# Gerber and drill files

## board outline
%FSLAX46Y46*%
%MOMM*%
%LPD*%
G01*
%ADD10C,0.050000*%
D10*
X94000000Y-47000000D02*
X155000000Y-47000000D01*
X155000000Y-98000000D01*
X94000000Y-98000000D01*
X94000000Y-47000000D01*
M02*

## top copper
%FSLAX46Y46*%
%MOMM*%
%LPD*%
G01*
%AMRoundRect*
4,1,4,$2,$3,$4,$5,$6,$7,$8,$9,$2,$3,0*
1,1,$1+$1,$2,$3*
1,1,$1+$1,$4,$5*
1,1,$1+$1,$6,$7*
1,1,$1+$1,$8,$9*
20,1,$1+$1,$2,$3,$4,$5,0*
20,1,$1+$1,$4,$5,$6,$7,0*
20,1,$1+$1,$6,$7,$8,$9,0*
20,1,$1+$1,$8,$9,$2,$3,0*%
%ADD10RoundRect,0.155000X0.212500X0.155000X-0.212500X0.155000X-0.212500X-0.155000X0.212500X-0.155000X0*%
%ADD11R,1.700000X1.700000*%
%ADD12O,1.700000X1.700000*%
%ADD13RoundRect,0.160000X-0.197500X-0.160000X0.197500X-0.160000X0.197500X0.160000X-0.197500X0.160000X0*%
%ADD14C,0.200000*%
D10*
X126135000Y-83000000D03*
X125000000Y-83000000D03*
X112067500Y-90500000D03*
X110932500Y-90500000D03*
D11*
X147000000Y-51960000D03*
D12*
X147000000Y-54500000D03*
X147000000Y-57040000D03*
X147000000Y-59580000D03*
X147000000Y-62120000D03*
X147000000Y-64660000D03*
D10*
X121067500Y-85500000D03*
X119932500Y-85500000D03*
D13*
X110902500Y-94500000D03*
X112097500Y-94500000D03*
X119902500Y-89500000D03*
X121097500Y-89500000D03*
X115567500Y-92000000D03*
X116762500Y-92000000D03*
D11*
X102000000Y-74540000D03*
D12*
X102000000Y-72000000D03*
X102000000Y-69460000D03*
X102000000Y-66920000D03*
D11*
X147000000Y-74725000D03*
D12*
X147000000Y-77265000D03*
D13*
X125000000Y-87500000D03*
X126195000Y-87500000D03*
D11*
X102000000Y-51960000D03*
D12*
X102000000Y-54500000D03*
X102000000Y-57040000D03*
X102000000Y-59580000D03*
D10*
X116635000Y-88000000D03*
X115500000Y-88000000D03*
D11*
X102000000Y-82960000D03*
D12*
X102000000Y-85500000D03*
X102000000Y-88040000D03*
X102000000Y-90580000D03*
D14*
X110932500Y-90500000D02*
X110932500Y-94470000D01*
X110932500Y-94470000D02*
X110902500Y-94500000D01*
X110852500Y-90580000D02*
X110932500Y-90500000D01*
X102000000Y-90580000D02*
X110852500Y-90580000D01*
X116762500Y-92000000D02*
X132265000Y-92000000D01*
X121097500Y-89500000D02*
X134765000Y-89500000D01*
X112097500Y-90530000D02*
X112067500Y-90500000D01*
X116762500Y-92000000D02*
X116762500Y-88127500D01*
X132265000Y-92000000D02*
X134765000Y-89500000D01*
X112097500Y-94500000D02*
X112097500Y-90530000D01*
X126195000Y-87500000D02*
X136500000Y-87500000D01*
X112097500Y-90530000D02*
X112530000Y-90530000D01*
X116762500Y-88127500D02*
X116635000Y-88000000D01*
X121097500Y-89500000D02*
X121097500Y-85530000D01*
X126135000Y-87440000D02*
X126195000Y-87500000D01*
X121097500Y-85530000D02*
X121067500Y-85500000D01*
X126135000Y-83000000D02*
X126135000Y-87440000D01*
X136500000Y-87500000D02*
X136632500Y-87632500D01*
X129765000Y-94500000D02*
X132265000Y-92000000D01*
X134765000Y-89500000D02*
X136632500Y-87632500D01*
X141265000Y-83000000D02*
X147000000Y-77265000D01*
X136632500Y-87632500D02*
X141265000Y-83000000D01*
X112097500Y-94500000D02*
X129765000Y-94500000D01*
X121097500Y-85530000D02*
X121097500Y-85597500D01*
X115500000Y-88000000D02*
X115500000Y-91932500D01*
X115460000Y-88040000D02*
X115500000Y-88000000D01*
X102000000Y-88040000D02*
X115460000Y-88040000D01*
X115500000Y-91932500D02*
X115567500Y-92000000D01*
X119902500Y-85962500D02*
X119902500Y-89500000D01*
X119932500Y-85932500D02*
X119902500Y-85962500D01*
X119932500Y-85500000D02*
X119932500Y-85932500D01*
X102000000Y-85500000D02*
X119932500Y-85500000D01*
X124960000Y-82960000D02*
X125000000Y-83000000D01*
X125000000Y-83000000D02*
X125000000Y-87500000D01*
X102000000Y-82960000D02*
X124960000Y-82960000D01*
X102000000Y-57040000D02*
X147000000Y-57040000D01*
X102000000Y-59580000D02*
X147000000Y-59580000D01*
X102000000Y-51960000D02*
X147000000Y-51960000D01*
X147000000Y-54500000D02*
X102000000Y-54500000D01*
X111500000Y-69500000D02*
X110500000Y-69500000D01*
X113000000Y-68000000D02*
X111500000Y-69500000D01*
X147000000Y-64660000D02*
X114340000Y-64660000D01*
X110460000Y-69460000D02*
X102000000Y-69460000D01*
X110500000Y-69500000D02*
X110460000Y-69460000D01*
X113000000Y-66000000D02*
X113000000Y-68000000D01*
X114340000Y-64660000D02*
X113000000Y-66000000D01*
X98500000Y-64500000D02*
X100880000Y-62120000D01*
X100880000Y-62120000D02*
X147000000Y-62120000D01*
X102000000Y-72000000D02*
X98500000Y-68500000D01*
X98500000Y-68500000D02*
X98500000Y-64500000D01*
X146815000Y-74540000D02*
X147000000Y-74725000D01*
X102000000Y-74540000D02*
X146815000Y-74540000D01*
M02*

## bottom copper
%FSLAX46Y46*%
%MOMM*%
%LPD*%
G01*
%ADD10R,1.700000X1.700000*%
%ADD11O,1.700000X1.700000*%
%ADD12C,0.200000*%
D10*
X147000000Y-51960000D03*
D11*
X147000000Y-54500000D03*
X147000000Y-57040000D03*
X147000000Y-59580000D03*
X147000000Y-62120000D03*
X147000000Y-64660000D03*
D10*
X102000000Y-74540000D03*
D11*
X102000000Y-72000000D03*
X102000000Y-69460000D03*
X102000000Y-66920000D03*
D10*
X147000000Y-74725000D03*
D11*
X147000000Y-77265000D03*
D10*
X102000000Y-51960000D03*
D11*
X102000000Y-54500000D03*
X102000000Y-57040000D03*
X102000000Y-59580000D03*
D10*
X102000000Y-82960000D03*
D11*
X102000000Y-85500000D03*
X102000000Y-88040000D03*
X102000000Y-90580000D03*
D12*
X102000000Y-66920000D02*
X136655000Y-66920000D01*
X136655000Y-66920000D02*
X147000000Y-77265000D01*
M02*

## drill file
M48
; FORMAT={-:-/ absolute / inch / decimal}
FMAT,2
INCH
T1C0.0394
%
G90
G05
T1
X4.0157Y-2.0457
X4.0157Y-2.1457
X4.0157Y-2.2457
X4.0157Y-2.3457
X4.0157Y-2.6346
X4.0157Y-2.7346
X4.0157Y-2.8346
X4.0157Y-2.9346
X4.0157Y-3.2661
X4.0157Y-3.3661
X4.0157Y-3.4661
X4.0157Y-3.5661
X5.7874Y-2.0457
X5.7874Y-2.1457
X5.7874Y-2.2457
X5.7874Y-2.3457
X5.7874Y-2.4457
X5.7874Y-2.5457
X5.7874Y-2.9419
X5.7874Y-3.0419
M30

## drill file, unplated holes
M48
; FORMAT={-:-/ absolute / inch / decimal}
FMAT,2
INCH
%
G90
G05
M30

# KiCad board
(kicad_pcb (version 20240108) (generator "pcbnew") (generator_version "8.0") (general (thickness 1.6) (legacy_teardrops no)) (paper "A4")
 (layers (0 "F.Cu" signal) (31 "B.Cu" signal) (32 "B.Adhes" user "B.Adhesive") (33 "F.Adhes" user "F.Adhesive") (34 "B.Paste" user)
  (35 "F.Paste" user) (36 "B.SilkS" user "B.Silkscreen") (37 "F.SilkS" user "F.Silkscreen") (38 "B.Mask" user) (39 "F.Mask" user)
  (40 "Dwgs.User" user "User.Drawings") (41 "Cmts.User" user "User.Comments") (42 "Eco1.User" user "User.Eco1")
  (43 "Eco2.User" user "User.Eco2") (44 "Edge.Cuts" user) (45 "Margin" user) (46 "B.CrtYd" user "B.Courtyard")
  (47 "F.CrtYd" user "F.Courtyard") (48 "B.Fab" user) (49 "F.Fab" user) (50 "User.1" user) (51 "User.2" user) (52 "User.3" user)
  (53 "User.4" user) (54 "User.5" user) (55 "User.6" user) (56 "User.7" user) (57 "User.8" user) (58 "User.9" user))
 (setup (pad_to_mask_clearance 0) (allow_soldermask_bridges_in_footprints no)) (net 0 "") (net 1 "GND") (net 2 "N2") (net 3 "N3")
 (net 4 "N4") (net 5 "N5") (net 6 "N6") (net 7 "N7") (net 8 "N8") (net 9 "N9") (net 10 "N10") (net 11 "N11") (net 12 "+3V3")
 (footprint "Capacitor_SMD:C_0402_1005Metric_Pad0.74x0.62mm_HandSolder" (layer "F.Cu") (at 125.5675 83 180)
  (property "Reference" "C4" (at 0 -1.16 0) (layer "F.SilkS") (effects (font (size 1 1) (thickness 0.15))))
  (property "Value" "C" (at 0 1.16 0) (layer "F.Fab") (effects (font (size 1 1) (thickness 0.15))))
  (pad "1" smd roundrect (at -0.5675 0 180) (size 0.735 0.62) (layers "F.Cu" "F.Paste" "F.Mask") (roundrect_rratio 0.25) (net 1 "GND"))
  (pad "2" smd roundrect (at 0.5675 0 180) (size 0.735 0.62) (layers "F.Cu" "F.Paste" "F.Mask") (roundrect_rratio 0.25) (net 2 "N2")))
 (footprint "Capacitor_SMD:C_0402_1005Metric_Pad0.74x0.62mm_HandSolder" (layer "F.Cu") (at 111.5 90.5 180)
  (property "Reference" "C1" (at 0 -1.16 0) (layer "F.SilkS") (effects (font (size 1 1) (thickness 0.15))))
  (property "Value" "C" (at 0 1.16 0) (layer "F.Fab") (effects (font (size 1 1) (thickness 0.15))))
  (pad "1" smd roundrect (at -0.5675 0 180) (size 0.735 0.62) (layers "F.Cu" "F.Paste" "F.Mask") (roundrect_rratio 0.25) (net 1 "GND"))
  (pad "2" smd roundrect (at 0.5675 0 180) (size 0.735 0.62) (layers "F.Cu" "F.Paste" "F.Mask") (roundrect_rratio 0.25) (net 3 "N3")))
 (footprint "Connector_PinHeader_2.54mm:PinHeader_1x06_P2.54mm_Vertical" (layer "F.Cu") (at 147 51.96)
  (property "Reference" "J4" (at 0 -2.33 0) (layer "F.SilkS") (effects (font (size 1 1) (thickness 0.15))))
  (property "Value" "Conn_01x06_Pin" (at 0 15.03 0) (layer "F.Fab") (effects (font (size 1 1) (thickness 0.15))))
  (pad "1" thru_hole rect (at 0 0) (size 1.7 1.7) (drill 1) (layers "*.Cu" "*.Mask") (remove_unused_layers no) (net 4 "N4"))
  (pad "2" thru_hole oval (at 0 2.54) (size 1.7 1.7) (drill 1) (layers "*.Cu" "*.Mask") (remove_unused_layers no) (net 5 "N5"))
  (pad "3" thru_hole oval (at 0 5.08) (size 1.7 1.7) (drill 1) (layers "*.Cu" "*.Mask") (remove_unused_layers no) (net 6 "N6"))
  (pad "4" thru_hole oval (at 0 7.62) (size 1.7 1.7) (drill 1) (layers "*.Cu" "*.Mask") (remove_unused_layers no) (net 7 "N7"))
  (pad "5" thru_hole oval (at 0 10.16) (size 1.7 1.7) (drill 1) (layers "*.Cu" "*.Mask") (remove_unused_layers no) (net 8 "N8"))
  (pad "6" thru_hole oval (at 0 12.7) (size 1.7 1.7) (drill 1) (layers "*.Cu" "*.Mask") (remove_unused_layers no) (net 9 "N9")))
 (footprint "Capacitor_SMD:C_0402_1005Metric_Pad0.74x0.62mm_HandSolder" (layer "F.Cu") (at 120.5 85.5 180)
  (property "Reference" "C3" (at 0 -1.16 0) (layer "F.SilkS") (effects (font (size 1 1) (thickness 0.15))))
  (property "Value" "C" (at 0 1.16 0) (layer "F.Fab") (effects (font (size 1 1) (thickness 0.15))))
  (pad "1" smd roundrect (at -0.5675 0 180) (size 0.735 0.62) (layers "F.Cu" "F.Paste" "F.Mask") (roundrect_rratio 0.25) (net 1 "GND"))
  (pad "2" smd roundrect (at 0.5675 0 180) (size 0.735 0.62) (layers "F.Cu" "F.Paste" "F.Mask") (roundrect_rratio 0.25) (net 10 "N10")))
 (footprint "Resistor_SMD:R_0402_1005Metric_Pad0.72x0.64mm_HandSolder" (layer "F.Cu") (at 111.5 94.5)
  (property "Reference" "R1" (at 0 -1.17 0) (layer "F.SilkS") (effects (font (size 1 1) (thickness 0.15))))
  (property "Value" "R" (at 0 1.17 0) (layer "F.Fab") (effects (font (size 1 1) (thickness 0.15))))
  (pad "1" smd roundrect (at -0.5975 0) (size 0.715 0.64) (layers "F.Cu" "F.Paste" "F.Mask") (roundrect_rratio 0.25) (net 3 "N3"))
  (pad "2" smd roundrect (at 0.5975 0) (size 0.715 0.64) (layers "F.Cu" "F.Paste" "F.Mask") (roundrect_rratio 0.25) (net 1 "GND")))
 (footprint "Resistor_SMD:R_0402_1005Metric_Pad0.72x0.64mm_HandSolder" (layer "F.Cu") (at 120.5 89.5)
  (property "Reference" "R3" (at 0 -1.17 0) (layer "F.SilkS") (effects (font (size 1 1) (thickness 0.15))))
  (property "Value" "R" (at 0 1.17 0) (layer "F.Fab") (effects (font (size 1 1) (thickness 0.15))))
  (pad "1" smd roundrect (at -0.5975 0) (size 0.715 0.64) (layers "F.Cu" "F.Paste" "F.Mask") (roundrect_rratio 0.25) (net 10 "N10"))
  (pad "2" smd roundrect (at 0.5975 0) (size 0.715 0.64) (layers "F.Cu" "F.Paste" "F.Mask") (roundrect_rratio 0.25) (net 1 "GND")))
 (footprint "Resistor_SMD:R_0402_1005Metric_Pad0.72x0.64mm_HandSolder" (layer "F.Cu") (at 116.165 92)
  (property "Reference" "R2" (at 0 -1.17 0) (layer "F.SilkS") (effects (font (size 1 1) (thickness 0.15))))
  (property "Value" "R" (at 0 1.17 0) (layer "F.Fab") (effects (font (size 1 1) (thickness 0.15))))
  (pad "1" smd roundrect (at -0.5975 0) (size 0.715 0.64) (layers "F.Cu" "F.Paste" "F.Mask") (roundrect_rratio 0.25) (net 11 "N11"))
  (pad "2" smd roundrect (at 0.5975 0) (size 0.715 0.64) (layers "F.Cu" "F.Paste" "F.Mask") (roundrect_rratio 0.25) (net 1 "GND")))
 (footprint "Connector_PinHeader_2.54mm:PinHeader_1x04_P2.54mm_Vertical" (layer "F.Cu") (at 102 74.54 180)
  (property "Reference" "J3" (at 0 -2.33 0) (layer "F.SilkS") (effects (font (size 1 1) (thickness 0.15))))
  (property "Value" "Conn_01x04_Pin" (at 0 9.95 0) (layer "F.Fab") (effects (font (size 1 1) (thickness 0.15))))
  (pad "1" thru_hole rect (at 0 0 180) (size 1.7 1.7) (drill 1) (layers "*.Cu" "*.Mask") (remove_unused_layers no) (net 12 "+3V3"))
  (pad "2" thru_hole oval (at 0 2.54 180) (size 1.7 1.7) (drill 1) (layers "*.Cu" "*.Mask") (remove_unused_layers no) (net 8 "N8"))
  (pad "3" thru_hole oval (at 0 5.08 180) (size 1.7 1.7) (drill 1) (layers "*.Cu" "*.Mask") (remove_unused_layers no) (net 9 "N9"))
  (pad "4" thru_hole oval (at 0 7.62 180) (size 1.7 1.7) (drill 1) (layers "*.Cu" "*.Mask") (remove_unused_layers no) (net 1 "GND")))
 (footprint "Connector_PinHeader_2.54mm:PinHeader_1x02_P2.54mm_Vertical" (layer "F.Cu") (at 147 74.725)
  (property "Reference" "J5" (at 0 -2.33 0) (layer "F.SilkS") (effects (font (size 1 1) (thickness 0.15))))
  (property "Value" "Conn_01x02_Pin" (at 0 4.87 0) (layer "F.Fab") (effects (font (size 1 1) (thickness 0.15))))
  (pad "1" thru_hole rect (at 0 0) (size 1.7 1.7) (drill 1) (layers "*.Cu" "*.Mask") (remove_unused_layers no) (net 12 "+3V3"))
  (pad "2" thru_hole oval (at 0 2.54) (size 1.7 1.7) (drill 1) (layers "*.Cu" "*.Mask") (remove_unused_layers no) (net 1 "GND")))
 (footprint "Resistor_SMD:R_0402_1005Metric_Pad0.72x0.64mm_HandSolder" (layer "F.Cu") (at 125.5975 87.5)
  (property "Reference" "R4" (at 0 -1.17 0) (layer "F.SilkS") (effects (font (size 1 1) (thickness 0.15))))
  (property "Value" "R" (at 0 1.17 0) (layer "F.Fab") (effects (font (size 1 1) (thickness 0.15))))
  (pad "1" smd roundrect (at -0.5975 0) (size 0.715 0.64) (layers "F.Cu" "F.Paste" "F.Mask") (roundrect_rratio 0.25) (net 2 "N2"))
  (pad "2" smd roundrect (at 0.5975 0) (size 0.715 0.64) (layers "F.Cu" "F.Paste" "F.Mask") (roundrect_rratio 0.25) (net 1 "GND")))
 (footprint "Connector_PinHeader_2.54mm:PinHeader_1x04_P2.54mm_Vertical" (layer "F.Cu") (at 102 51.96)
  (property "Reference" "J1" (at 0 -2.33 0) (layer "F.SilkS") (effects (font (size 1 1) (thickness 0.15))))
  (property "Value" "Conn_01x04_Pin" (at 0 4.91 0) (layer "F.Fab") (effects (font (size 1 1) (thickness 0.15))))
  (pad "1" thru_hole rect (at 0 0) (size 1.7 1.7) (drill 1) (layers "*.Cu" "*.Mask") (remove_unused_layers no) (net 4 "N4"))
  (pad "2" thru_hole oval (at 0 2.54) (size 1.7 1.7) (drill 1) (layers "*.Cu" "*.Mask") (remove_unused_layers no) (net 5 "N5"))
  (pad "3" thru_hole oval (at 0 5.08) (size 1.7 1.7) (drill 1) (layers "*.Cu" "*.Mask") (remove_unused_layers no) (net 6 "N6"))
  (pad "4" thru_hole oval (at 0 7.62) (size 1.7 1.7) (drill 1) (layers "*.Cu" "*.Mask") (remove_unused_layers no) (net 7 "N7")))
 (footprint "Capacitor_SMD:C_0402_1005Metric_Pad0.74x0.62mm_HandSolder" (layer "F.Cu") (at 116.0675 88 180)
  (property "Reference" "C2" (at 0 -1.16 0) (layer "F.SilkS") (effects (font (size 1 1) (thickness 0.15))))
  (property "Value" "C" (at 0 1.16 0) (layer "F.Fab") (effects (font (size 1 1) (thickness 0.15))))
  (pad "1" smd roundrect (at -0.5675 0 180) (size 0.735 0.62) (layers "F.Cu" "F.Paste" "F.Mask") (roundrect_rratio 0.25) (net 1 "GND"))
  (pad "2" smd roundrect (at 0.5675 0 180) (size 0.735 0.62) (layers "F.Cu" "F.Paste" "F.Mask") (roundrect_rratio 0.25) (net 11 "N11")))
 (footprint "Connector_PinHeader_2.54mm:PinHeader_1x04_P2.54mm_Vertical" (layer "F.Cu") (at 102 82.96)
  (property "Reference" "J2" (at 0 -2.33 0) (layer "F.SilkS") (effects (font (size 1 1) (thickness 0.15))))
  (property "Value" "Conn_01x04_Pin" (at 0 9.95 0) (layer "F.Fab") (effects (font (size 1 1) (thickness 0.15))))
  (pad "1" thru_hole rect (at 0 0) (size 1.7 1.7) (drill 1) (layers "*.Cu" "*.Mask") (remove_unused_layers no) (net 2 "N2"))
  (pad "2" thru_hole oval (at 0 2.54) (size 1.7 1.7) (drill 1) (layers "*.Cu" "*.Mask") (remove_unused_layers no) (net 10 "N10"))
  (pad "3" thru_hole oval (at 0 5.08) (size 1.7 1.7) (drill 1) (layers "*.Cu" "*.Mask") (remove_unused_layers no) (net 11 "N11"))
  (pad "4" thru_hole oval (at 0 7.62) (size 1.7 1.7) (drill 1) (layers "*.Cu" "*.Mask") (remove_unused_layers no) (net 3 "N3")))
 (gr_rect (start 94 47) (end 155 98) (stroke (width 0.05) (type default)) (fill none) (layer "Edge.Cuts"))
 (segment (start 110.9325 90.5) (end 110.9325 94.47) (width 0.2) (layer "F.Cu") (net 3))
 (segment (start 110.9325 94.47) (end 110.9025 94.5) (width 0.2) (layer "F.Cu") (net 3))
 (segment (start 110.8525 90.58) (end 110.9325 90.5) (width 0.2) (layer "F.Cu") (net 3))
 (segment (start 102 90.58) (end 110.8525 90.58) (width 0.2) (layer "F.Cu") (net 3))
 (segment (start 116.7625 92) (end 132.265 92) (width 0.2) (layer "F.Cu") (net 1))
 (segment (start 121.0975 89.5) (end 134.765 89.5) (width 0.2) (layer "F.Cu") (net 1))
 (segment (start 112.0975 90.53) (end 112.0675 90.5) (width 0.2) (layer "F.Cu") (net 1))
 (segment (start 116.7625 92) (end 116.7625 88.1275) (width 0.2) (layer "F.Cu") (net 1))
 (segment (start 132.265 92) (end 134.765 89.5) (width 0.2) (layer "F.Cu") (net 1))
 (segment (start 112.0975 94.5) (end 112.0975 90.53) (width 0.2) (layer "F.Cu") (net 1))
 (segment (start 126.195 87.5) (end 136.5 87.5) (width 0.2) (layer "F.Cu") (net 1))
 (segment (start 112.0975 90.53) (end 112.53 90.53) (width 0.2) (layer "F.Cu") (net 1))
 (segment (start 116.7625 88.1275) (end 116.635 88) (width 0.2) (layer "F.Cu") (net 1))
 (segment (start 121.0975 89.5) (end 121.0975 85.53) (width 0.2) (layer "F.Cu") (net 1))
 (segment (start 126.135 87.44) (end 126.195 87.5) (width 0.2) (layer "F.Cu") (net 1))
 (segment (start 121.0975 85.53) (end 121.0675 85.5) (width 0.2) (layer "F.Cu") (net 1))
 (segment (start 126.135 83) (end 126.135 87.44) (width 0.2) (layer "F.Cu") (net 1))
 (segment (start 136.5 87.5) (end 136.6325 87.6325) (width 0.2) (layer "F.Cu") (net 1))
 (segment (start 129.765 94.5) (end 132.265 92) (width 0.2) (layer "F.Cu") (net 1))
 (segment (start 134.765 89.5) (end 136.6325 87.6325) (width 0.2) (layer "F.Cu") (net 1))
 (segment (start 141.265 83) (end 147 77.265) (width 0.2) (layer "F.Cu") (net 1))
 (segment (start 136.6325 87.6325) (end 141.265 83) (width 0.2) (layer "F.Cu") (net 1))
 (segment (start 112.0975 94.5) (end 129.765 94.5) (width 0.2) (layer "F.Cu") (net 1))
 (segment (start 121.0975 85.53) (end 121.0975 85.5975) (width 0.2) (layer "F.Cu") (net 1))
 (segment (start 102 66.92) (end 136.655 66.92) (width 0.2) (layer "B.Cu") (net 1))
 (segment (start 136.655 66.92) (end 147 77.265) (width 0.2) (layer "B.Cu") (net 1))
 (segment (start 115.5 88) (end 115.5 91.9325) (width 0.2) (layer "F.Cu") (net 11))
 (segment (start 115.46 88.04) (end 115.5 88) (width 0.2) (layer "F.Cu") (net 11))
 (segment (start 102 88.04) (end 115.46 88.04) (width 0.2) (layer "F.Cu") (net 11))
 (segment (start 115.5 91.9325) (end 115.5675 92) (width 0.2) (layer "F.Cu") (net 11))
 (segment (start 119.9025 85.9625) (end 119.9025 89.5) (width 0.2) (layer "F.Cu") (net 10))
 (segment (start 119.9325 85.9325) (end 119.9025 85.9625) (width 0.2) (layer "F.Cu") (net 10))
 (segment (start 119.9325 85.5) (end 119.9325 85.9325) (width 0.2) (layer "F.Cu") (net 10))
 (segment (start 102 85.5) (end 119.9325 85.5) (width 0.2) (layer "F.Cu") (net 10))
 (segment (start 124.96 82.96) (end 125 83) (width 0.2) (layer "F.Cu") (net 2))
 (segment (start 125 83) (end 125 87.5) (width 0.2) (layer "F.Cu") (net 2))
 (segment (start 102 82.96) (end 124.96 82.96) (width 0.2) (layer "F.Cu") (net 2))
 (segment (start 102 57.04) (end 147 57.04) (width 0.2) (layer "F.Cu") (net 6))
 (segment (start 102 59.58) (end 147 59.58) (width 0.2) (layer "F.Cu") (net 7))
 (segment (start 102 51.96) (end 147 51.96) (width 0.2) (layer "F.Cu") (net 4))
 (segment (start 147 54.5) (end 102 54.5) (width 0.2) (layer "F.Cu") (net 5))
 (segment (start 111.5 69.5) (end 110.5 69.5) (width 0.2) (layer "F.Cu") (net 9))
 (segment (start 113 68) (end 111.5 69.5) (width 0.2) (layer "F.Cu") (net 9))
 (segment (start 147 64.66) (end 114.34 64.66) (width 0.2) (layer "F.Cu") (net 9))
 (segment (start 110.46 69.46) (end 102 69.46) (width 0.2) (layer "F.Cu") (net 9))
 (segment (start 110.5 69.5) (end 110.46 69.46) (width 0.2) (layer "F.Cu") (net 9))
 (segment (start 113 66) (end 113 68) (width 0.2) (layer "F.Cu") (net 9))
 (segment (start 114.34 64.66) (end 113 66) (width 0.2) (layer "F.Cu") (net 9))
 (segment (start 98.5 64.5) (end 100.88 62.12) (width 0.2) (layer "F.Cu") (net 8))
 (segment (start 100.88 62.12) (end 147 62.12) (width 0.2) (layer "F.Cu") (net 8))
 (segment (start 102 72) (end 98.5 68.5) (width 0.2) (layer "F.Cu") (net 8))
 (segment (start 98.5 68.5) (end 98.5 64.5) (width 0.2) (layer "F.Cu") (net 8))
 (segment (start 146.815 74.54) (end 147 74.725) (width 0.2) (layer "F.Cu") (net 12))
 (segment (start 102 74.54) (end 146.815 74.54) (width 0.2) (layer "F.Cu") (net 12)))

